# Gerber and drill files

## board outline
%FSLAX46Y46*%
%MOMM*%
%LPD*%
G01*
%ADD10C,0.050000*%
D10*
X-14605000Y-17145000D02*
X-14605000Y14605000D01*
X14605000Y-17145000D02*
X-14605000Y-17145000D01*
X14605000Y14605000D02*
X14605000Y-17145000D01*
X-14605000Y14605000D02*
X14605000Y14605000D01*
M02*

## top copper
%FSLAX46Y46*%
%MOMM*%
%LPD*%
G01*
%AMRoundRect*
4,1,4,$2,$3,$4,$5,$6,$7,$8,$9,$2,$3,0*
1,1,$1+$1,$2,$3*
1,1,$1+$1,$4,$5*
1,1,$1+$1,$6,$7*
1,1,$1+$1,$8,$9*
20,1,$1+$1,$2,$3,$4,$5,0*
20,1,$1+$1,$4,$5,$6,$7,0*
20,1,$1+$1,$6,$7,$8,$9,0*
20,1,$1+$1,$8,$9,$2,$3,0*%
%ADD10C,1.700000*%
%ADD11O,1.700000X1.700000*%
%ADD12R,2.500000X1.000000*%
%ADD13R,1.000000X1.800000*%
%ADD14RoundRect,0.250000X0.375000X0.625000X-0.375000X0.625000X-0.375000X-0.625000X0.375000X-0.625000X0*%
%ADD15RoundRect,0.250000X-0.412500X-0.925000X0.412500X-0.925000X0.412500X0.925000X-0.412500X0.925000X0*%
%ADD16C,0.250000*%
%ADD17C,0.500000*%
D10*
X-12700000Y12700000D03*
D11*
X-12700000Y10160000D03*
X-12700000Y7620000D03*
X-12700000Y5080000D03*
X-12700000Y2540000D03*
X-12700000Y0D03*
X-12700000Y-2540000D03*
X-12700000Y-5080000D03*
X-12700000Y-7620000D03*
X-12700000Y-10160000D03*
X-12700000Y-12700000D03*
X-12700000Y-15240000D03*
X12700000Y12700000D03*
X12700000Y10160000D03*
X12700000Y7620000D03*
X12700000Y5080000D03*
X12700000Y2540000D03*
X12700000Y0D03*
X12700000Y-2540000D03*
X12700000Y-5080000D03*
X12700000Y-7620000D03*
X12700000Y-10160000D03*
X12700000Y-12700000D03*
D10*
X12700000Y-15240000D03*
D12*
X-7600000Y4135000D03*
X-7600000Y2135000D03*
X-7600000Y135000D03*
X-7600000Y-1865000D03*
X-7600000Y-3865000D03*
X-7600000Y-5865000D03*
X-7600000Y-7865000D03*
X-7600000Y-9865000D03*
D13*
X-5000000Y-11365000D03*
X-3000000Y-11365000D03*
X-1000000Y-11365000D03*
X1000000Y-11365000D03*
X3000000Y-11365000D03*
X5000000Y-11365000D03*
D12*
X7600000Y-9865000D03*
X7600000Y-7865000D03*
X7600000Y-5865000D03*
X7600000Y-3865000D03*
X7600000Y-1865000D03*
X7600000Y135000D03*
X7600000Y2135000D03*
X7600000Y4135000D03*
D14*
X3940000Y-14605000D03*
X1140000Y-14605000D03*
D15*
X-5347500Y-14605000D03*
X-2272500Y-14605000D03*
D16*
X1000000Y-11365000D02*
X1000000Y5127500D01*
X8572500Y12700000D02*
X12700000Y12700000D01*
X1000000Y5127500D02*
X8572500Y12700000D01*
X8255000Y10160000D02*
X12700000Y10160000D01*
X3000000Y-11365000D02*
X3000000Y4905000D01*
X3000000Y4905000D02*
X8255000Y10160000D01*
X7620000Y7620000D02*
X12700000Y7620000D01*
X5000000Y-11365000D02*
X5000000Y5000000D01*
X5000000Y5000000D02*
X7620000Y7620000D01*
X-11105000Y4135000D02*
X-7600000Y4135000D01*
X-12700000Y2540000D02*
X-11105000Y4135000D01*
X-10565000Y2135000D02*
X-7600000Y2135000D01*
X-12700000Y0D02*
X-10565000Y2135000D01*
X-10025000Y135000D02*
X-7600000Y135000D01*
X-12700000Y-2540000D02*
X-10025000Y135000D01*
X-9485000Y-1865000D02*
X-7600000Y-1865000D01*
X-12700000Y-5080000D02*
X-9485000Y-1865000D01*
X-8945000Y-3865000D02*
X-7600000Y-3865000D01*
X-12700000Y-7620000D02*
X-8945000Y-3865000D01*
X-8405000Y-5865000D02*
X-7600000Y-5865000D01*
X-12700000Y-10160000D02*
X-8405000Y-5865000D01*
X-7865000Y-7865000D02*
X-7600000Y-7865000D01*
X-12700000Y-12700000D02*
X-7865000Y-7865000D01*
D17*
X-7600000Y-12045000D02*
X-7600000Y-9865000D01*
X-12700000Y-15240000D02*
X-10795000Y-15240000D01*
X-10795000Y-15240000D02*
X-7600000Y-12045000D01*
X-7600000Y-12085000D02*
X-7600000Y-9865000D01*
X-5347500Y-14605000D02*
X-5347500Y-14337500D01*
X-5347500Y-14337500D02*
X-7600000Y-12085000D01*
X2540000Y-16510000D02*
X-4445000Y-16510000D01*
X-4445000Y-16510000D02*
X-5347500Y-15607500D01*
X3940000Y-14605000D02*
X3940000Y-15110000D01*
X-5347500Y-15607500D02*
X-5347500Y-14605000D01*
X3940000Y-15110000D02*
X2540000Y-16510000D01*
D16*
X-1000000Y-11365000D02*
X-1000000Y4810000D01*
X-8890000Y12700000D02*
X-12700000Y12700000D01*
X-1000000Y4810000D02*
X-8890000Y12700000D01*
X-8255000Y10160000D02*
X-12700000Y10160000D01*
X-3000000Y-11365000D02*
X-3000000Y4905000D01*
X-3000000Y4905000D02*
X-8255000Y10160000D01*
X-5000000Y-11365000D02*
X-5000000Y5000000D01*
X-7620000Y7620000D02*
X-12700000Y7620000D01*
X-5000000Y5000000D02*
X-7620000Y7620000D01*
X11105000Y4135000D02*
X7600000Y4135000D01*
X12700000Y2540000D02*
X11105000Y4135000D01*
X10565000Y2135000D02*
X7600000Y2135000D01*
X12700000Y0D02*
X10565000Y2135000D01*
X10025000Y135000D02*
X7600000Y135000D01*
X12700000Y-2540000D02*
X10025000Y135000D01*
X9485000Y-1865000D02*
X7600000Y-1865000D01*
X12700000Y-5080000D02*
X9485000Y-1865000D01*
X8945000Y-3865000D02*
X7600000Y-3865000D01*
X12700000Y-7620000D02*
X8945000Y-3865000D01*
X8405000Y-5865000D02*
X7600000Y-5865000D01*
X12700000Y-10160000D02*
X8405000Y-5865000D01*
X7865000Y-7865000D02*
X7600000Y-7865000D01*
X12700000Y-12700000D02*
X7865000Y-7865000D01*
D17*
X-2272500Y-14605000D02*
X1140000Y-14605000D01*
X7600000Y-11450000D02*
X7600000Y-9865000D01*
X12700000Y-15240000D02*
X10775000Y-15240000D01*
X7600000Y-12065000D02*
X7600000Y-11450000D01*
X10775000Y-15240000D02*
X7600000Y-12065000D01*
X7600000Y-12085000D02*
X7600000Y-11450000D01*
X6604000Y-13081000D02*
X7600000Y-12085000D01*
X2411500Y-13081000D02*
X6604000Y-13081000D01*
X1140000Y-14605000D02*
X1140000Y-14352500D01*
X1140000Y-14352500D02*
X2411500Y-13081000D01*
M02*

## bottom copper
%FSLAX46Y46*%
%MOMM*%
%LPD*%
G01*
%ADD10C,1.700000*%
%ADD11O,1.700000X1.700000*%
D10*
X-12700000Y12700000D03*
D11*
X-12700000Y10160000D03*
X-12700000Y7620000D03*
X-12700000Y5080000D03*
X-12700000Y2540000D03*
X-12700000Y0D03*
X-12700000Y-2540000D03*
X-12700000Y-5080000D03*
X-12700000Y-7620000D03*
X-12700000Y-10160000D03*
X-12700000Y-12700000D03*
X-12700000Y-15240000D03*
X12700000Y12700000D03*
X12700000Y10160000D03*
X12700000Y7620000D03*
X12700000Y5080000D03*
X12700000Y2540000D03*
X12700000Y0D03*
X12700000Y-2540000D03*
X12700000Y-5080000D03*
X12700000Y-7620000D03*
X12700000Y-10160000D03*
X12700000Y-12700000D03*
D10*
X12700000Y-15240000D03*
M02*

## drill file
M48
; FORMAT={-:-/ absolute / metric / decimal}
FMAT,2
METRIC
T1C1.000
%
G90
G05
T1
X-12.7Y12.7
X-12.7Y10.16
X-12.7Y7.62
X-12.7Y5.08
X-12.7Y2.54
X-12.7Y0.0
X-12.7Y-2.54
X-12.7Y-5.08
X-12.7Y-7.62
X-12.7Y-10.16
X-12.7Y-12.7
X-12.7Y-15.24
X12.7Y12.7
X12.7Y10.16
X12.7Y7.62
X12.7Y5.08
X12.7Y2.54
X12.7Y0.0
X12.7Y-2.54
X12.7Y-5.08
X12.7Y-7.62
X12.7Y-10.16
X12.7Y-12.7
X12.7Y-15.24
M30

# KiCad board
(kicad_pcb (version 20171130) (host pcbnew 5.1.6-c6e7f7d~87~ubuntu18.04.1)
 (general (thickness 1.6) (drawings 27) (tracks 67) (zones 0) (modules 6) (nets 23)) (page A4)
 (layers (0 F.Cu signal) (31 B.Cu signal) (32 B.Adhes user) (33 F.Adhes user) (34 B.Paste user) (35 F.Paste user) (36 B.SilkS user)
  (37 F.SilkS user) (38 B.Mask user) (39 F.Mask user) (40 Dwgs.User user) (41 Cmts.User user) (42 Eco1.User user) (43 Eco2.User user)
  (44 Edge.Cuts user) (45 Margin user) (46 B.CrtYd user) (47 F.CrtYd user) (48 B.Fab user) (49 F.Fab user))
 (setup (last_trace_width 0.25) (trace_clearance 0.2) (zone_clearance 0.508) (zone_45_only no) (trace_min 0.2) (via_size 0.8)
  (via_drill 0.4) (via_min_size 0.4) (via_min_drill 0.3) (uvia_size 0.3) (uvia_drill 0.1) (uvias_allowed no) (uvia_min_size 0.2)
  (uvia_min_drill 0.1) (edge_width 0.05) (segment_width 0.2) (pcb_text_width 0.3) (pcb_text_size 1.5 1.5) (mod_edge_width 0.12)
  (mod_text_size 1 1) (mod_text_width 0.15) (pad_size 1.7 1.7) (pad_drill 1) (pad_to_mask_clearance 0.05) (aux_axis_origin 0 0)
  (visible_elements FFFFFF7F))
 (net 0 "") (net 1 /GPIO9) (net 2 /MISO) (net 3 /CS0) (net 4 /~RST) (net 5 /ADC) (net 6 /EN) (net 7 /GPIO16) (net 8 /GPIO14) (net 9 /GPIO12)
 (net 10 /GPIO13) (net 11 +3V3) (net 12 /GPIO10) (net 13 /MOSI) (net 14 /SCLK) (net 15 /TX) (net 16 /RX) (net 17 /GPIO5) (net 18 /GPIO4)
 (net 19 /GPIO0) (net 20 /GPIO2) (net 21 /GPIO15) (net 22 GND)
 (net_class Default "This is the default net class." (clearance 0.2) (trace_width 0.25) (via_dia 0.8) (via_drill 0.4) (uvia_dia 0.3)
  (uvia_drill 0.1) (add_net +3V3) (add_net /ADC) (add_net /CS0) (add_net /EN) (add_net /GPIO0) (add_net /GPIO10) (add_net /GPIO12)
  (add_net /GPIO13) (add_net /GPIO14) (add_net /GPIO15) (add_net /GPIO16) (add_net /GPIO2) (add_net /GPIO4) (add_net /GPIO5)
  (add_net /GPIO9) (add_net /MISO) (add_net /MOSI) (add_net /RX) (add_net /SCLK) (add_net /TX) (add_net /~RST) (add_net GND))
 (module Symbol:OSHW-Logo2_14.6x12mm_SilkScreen (layer B.Cu) (at 0 3.81 180)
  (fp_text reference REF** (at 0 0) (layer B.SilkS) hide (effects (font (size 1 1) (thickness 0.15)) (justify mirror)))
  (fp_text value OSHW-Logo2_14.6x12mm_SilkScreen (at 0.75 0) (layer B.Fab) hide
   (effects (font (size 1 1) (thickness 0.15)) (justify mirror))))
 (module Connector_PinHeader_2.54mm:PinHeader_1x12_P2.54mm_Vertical (layer B.Cu) (at -12.7 -12.7 180)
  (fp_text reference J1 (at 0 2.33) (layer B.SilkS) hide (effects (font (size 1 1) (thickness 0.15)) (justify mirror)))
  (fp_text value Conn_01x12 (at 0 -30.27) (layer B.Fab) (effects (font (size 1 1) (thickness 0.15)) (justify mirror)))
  (pad 1 thru_hole circle (at 0 0 180) (size 1.7 1.7) (drill 1) (layers *.Cu *.Mask) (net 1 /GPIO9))
  (pad 2 thru_hole oval (at 0 -2.54 180) (size 1.7 1.7) (drill 1) (layers *.Cu *.Mask) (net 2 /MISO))
  (pad 3 thru_hole oval (at 0 -5.08 180) (size 1.7 1.7) (drill 1) (layers *.Cu *.Mask) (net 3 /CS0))
  (pad 4 thru_hole oval (at 0 -7.62 180) (size 1.7 1.7) (drill 1) (layers *.Cu *.Mask))
  (pad 5 thru_hole oval (at 0 -10.16 180) (size 1.7 1.7) (drill 1) (layers *.Cu *.Mask) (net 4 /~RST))
  (pad 6 thru_hole oval (at 0 -12.7 180) (size 1.7 1.7) (drill 1) (layers *.Cu *.Mask) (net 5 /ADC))
  (pad 7 thru_hole oval (at 0 -15.24 180) (size 1.7 1.7) (drill 1) (layers *.Cu *.Mask) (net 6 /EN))
  (pad 8 thru_hole oval (at 0 -17.78 180) (size 1.7 1.7) (drill 1) (layers *.Cu *.Mask) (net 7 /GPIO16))
  (pad 9 thru_hole oval (at 0 -20.32 180) (size 1.7 1.7) (drill 1) (layers *.Cu *.Mask) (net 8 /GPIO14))
  (pad 10 thru_hole oval (at 0 -22.86 180) (size 1.7 1.7) (drill 1) (layers *.Cu *.Mask) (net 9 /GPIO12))
  (pad 11 thru_hole oval (at 0 -25.4 180) (size 1.7 1.7) (drill 1) (layers *.Cu *.Mask) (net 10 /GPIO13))
  (pad 12 thru_hole oval (at 0 -27.94 180) (size 1.7 1.7) (drill 1) (layers *.Cu *.Mask) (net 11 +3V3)))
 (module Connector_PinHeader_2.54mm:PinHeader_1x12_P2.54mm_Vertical (layer B.Cu) (at 12.7 15.24)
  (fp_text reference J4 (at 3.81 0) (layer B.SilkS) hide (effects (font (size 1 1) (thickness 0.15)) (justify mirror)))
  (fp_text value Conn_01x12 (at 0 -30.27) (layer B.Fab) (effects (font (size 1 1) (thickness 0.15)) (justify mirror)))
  (pad 12 thru_hole oval (at 0 -27.94) (size 1.7 1.7) (drill 1) (layers *.Cu *.Mask) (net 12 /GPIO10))
  (pad 11 thru_hole oval (at 0 -25.4) (size 1.7 1.7) (drill 1) (layers *.Cu *.Mask) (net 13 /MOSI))
  (pad 10 thru_hole oval (at 0 -22.86) (size 1.7 1.7) (drill 1) (layers *.Cu *.Mask) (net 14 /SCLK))
  (pad 9 thru_hole oval (at 0 -20.32) (size 1.7 1.7) (drill 1) (layers *.Cu *.Mask))
  (pad 8 thru_hole oval (at 0 -17.78) (size 1.7 1.7) (drill 1) (layers *.Cu *.Mask) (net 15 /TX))
  (pad 7 thru_hole oval (at 0 -15.24) (size 1.7 1.7) (drill 1) (layers *.Cu *.Mask) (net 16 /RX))
  (pad 6 thru_hole oval (at 0 -12.7) (size 1.7 1.7) (drill 1) (layers *.Cu *.Mask) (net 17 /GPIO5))
  (pad 5 thru_hole oval (at 0 -10.16) (size 1.7 1.7) (drill 1) (layers *.Cu *.Mask) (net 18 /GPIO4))
  (pad 4 thru_hole oval (at 0 -7.62) (size 1.7 1.7) (drill 1) (layers *.Cu *.Mask) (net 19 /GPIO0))
  (pad 3 thru_hole oval (at 0 -5.08) (size 1.7 1.7) (drill 1) (layers *.Cu *.Mask) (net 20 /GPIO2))
  (pad 2 thru_hole oval (at 0 -2.54) (size 1.7 1.7) (drill 1) (layers *.Cu *.Mask) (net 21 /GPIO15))
  (pad 1 thru_hole circle (at 0 0) (size 1.7 1.7) (drill 1) (layers *.Cu *.Mask) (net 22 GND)))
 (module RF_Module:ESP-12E (layer F.Cu) (at 0 -0.635)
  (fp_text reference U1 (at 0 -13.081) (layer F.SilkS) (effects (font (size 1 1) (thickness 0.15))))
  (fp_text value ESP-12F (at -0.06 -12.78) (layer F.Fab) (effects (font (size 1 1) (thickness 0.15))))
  (pad 1 smd rect (at -7.6 -3.5) (size 2.5 1) (layers F.Cu F.Paste F.Mask) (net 4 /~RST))
  (pad 2 smd rect (at -7.6 -1.5) (size 2.5 1) (layers F.Cu F.Paste F.Mask) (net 5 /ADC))
  (pad 3 smd rect (at -7.6 0.5) (size 2.5 1) (layers F.Cu F.Paste F.Mask) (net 6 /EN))
  (pad 4 smd rect (at -7.6 2.5) (size 2.5 1) (layers F.Cu F.Paste F.Mask) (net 7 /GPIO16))
  (pad 5 smd rect (at -7.6 4.5) (size 2.5 1) (layers F.Cu F.Paste F.Mask) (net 8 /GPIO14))
  (pad 6 smd rect (at -7.6 6.5) (size 2.5 1) (layers F.Cu F.Paste F.Mask) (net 9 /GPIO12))
  (pad 7 smd rect (at -7.6 8.5) (size 2.5 1) (layers F.Cu F.Paste F.Mask) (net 10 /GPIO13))
  (pad 8 smd rect (at -7.6 10.5) (size 2.5 1) (layers F.Cu F.Paste F.Mask) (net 11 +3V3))
  (pad 9 smd rect (at -5 12) (size 1 1.8) (layers F.Cu F.Paste F.Mask) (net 3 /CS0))
  (pad 10 smd rect (at -3 12) (size 1 1.8) (layers F.Cu F.Paste F.Mask) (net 2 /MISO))
  (pad 11 smd rect (at -1 12) (size 1 1.8) (layers F.Cu F.Paste F.Mask) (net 1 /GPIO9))
  (pad 12 smd rect (at 1 12) (size 1 1.8) (layers F.Cu F.Paste F.Mask) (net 12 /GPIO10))
  (pad 13 smd rect (at 3 12) (size 1 1.8) (layers F.Cu F.Paste F.Mask) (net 13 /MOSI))
  (pad 14 smd rect (at 5 12) (size 1 1.8) (layers F.Cu F.Paste F.Mask) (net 14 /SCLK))
  (pad 15 smd rect (at 7.6 10.5) (size 2.5 1) (layers F.Cu F.Paste F.Mask) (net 22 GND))
  (pad 16 smd rect (at 7.6 8.5) (size 2.5 1) (layers F.Cu F.Paste F.Mask) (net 21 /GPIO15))
  (pad 17 smd rect (at 7.6 6.5) (size 2.5 1) (layers F.Cu F.Paste F.Mask) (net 20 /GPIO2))
  (pad 18 smd rect (at 7.6 4.5) (size 2.5 1) (layers F.Cu F.Paste F.Mask) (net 19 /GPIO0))
  (pad 19 smd rect (at 7.6 2.5) (size 2.5 1) (layers F.Cu F.Paste F.Mask) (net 18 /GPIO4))
  (pad 20 smd rect (at 7.6 0.5) (size 2.5 1) (layers F.Cu F.Paste F.Mask) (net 17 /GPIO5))
  (pad 21 smd rect (at 7.6 -1.5) (size 2.5 1) (layers F.Cu F.Paste F.Mask) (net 16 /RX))
  (pad 22 smd rect (at 7.6 -3.5) (size 2.5 1) (layers F.Cu F.Paste F.Mask) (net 15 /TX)))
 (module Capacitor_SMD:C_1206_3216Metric (layer F.Cu) (at 2.54 14.605 180)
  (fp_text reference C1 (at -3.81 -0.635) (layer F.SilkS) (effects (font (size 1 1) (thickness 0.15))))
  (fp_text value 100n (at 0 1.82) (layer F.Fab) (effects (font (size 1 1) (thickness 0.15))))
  (pad 1 smd roundrect (at -1.4 0 180) (size 1.25 1.75) (layers F.Cu F.Paste F.Mask) (roundrect_rratio 0.2) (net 11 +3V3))
  (pad 2 smd roundrect (at 1.4 0 180) (size 1.25 1.75) (layers F.Cu F.Paste F.Mask) (roundrect_rratio 0.2) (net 22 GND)))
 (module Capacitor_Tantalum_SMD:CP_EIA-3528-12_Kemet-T (layer F.Cu) (at -3.81 14.605)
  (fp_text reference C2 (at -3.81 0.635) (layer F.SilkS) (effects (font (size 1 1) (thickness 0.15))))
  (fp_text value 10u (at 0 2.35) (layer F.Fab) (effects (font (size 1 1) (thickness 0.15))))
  (pad 1 smd roundrect (at -1.5375 0) (size 1.325 2.35) (layers F.Cu F.Paste F.Mask) (roundrect_rratio 0.188679) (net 11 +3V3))
  (pad 2 smd roundrect (at 1.5375 0) (size 1.325 2.35) (layers F.Cu F.Paste F.Mask) (roundrect_rratio 0.188679) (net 22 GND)))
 (gr_line (start -14.605 17.145) (end -14.605 -14.605) (layer Edge.Cuts) (width 0.05))
 (gr_line (start 14.605 17.145) (end -14.605 17.145) (layer Edge.Cuts) (width 0.05))
 (gr_line (start 14.605 -14.605) (end 14.605 17.145) (layer Edge.Cuts) (width 0.05))
 (gr_line (start -14.605 -14.605) (end 14.605 -14.605) (layer Edge.Cuts) (width 0.05))
 (segment (start 1 11.365) (end 1 -5.1275) (width 0.25) (layer F.Cu) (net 12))
 (segment (start 8.5725 -12.7) (end 12.7 -12.7) (width 0.25) (layer F.Cu) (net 12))
 (segment (start 1 -5.1275) (end 8.5725 -12.7) (width 0.25) (layer F.Cu) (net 12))
 (segment (start 8.255 -10.16) (end 12.7 -10.16) (width 0.25) (layer F.Cu) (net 13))
 (segment (start 3 11.365) (end 3 -4.905) (width 0.25) (layer F.Cu) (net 13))
 (segment (start 3 -4.905) (end 8.255 -10.16) (width 0.25) (layer F.Cu) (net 13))
 (segment (start 7.62 -7.62) (end 12.7 -7.62) (width 0.25) (layer F.Cu) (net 14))
 (segment (start 5 11.365) (end 5 -5) (width 0.25) (layer F.Cu) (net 14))
 (segment (start 5 -5) (end 7.62 -7.62) (width 0.25) (layer F.Cu) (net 14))
 (segment (start -11.105 -4.135) (end -7.6 -4.135) (width 0.25) (layer F.Cu) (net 4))
 (segment (start -12.7 -2.54) (end -11.105 -4.135) (width 0.25) (layer F.Cu) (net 4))
 (segment (start -10.565 -2.135) (end -7.6 -2.135) (width 0.25) (layer F.Cu) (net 5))
 (segment (start -12.7 0) (end -10.565 -2.135) (width 0.25) (layer F.Cu) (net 5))
 (segment (start -10.025 -0.135) (end -7.6 -0.135) (width 0.25) (layer F.Cu) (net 6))
 (segment (start -12.7 2.54) (end -10.025 -0.135) (width 0.25) (layer F.Cu) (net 6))
 (segment (start -9.485 1.865) (end -7.6 1.865) (width 0.25) (layer F.Cu) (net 7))
 (segment (start -12.7 5.08) (end -9.485 1.865) (width 0.25) (layer F.Cu) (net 7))
 (segment (start -8.945 3.865) (end -7.6 3.865) (width 0.25) (layer F.Cu) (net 8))
 (segment (start -12.7 7.62) (end -8.945 3.865) (width 0.25) (layer F.Cu) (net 8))
 (segment (start -8.405 5.865) (end -7.6 5.865) (width 0.25) (layer F.Cu) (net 9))
 (segment (start -12.7 10.16) (end -8.405 5.865) (width 0.25) (layer F.Cu) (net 9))
 (segment (start -7.865 7.865) (end -7.6 7.865) (width 0.25) (layer F.Cu) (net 10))
 (segment (start -12.7 12.7) (end -7.865 7.865) (width 0.25) (layer F.Cu) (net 10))
 (segment (start -7.6 12.045) (end -7.6 9.865) (width 0.5) (layer F.Cu) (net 11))
 (segment (start -12.7 15.24) (end -10.795 15.24) (width 0.5) (layer F.Cu) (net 11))
 (segment (start -10.795 15.24) (end -7.6 12.045) (width 0.5) (layer F.Cu) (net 11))
 (segment (start -7.6 12.085) (end -7.6 9.865) (width 0.5) (layer F.Cu) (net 11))
 (segment (start -5.3475 14.605) (end -5.3475 14.3375) (width 0.5) (layer F.Cu) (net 11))
 (segment (start -5.3475 14.3375) (end -7.6 12.085) (width 0.5) (layer F.Cu) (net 11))
 (segment (start 2.54 16.51) (end -4.445 16.51) (width 0.5) (layer F.Cu) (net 11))
 (segment (start -4.445 16.51) (end -5.3475 15.6075) (width 0.5) (layer F.Cu) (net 11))
 (segment (start 3.94 14.605) (end 3.94 15.11) (width 0.5) (layer F.Cu) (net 11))
 (segment (start -5.3475 15.6075) (end -5.3475 14.605) (width 0.5) (layer F.Cu) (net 11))
 (segment (start 3.94 15.11) (end 2.54 16.51) (width 0.5) (layer F.Cu) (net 11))
 (segment (start -1 11.365) (end -1 -4.81) (width 0.25) (layer F.Cu) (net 1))
 (segment (start -8.89 -12.7) (end -12.7 -12.7) (width 0.25) (layer F.Cu) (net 1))
 (segment (start -1 -4.81) (end -8.89 -12.7) (width 0.25) (layer F.Cu) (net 1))
 (segment (start -8.255 -10.16) (end -12.7 -10.16) (width 0.25) (layer F.Cu) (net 2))
 (segment (start -3 11.365) (end -3 -4.905) (width 0.25) (layer F.Cu) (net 2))
 (segment (start -3 -4.905) (end -8.255 -10.16) (width 0.25) (layer F.Cu) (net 2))
 (segment (start -5 11.365) (end -5 -5) (width 0.25) (layer F.Cu) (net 3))
 (segment (start -7.62 -7.62) (end -12.7 -7.62) (width 0.25) (layer F.Cu) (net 3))
 (segment (start -5 -5) (end -7.62 -7.62) (width 0.25) (layer F.Cu) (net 3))
 (segment (start 11.105 -4.135) (end 7.6 -4.135) (width 0.25) (layer F.Cu) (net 15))
 (segment (start 12.7 -2.54) (end 11.105 -4.135) (width 0.25) (layer F.Cu) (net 15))
 (segment (start 10.565 -2.135) (end 7.6 -2.135) (width 0.25) (layer F.Cu) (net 16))
 (segment (start 12.7 0) (end 10.565 -2.135) (width 0.25) (layer F.Cu) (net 16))
 (segment (start 10.025 -0.135) (end 7.6 -0.135) (width 0.25) (layer F.Cu) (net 17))
 (segment (start 12.7 2.54) (end 10.025 -0.135) (width 0.25) (layer F.Cu) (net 17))
 (segment (start 9.485 1.865) (end 7.6 1.865) (width 0.25) (layer F.Cu) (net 18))
 (segment (start 12.7 5.08) (end 9.485 1.865) (width 0.25) (layer F.Cu) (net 18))
 (segment (start 8.945 3.865) (end 7.6 3.865) (width 0.25) (layer F.Cu) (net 19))
 (segment (start 12.7 7.62) (end 8.945 3.865) (width 0.25) (layer F.Cu) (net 19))
 (segment (start 8.405 5.865) (end 7.6 5.865) (width 0.25) (layer F.Cu) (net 20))
 (segment (start 12.7 10.16) (end 8.405 5.865) (width 0.25) (layer F.Cu) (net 20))
 (segment (start 7.865 7.865) (end 7.6 7.865) (width 0.25) (layer F.Cu) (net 21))
 (segment (start 12.7 12.7) (end 7.865 7.865) (width 0.25) (layer F.Cu) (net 21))
 (segment (start -2.2725 14.605) (end 1.14 14.605) (width 0.5) (layer F.Cu) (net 22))
 (segment (start 7.6 11.45) (end 7.6 9.865) (width 0.5) (layer F.Cu) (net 22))
 (segment (start 12.7 15.24) (end 10.775 15.24) (width 0.5) (layer F.Cu) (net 22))
 (segment (start 7.6 12.065) (end 7.6 11.45) (width 0.5) (layer F.Cu) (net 22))
 (segment (start 10.775 15.24) (end 7.6 12.065) (width 0.5) (layer F.Cu) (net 22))
 (segment (start 7.6 12.085) (end 7.6 11.45) (width 0.5) (layer F.Cu) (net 22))
 (segment (start 6.604 13.081) (end 7.6 12.085) (width 0.5) (layer F.Cu) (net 22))
 (segment (start 2.4115 13.081) (end 6.604 13.081) (width 0.5) (layer F.Cu) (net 22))
 (segment (start 1.14 14.605) (end 1.14 14.3525) (width 0.5) (layer F.Cu) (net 22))
 (segment (start 1.14 14.3525) (end 2.4115 13.081) (width 0.5) (layer F.Cu) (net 22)))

